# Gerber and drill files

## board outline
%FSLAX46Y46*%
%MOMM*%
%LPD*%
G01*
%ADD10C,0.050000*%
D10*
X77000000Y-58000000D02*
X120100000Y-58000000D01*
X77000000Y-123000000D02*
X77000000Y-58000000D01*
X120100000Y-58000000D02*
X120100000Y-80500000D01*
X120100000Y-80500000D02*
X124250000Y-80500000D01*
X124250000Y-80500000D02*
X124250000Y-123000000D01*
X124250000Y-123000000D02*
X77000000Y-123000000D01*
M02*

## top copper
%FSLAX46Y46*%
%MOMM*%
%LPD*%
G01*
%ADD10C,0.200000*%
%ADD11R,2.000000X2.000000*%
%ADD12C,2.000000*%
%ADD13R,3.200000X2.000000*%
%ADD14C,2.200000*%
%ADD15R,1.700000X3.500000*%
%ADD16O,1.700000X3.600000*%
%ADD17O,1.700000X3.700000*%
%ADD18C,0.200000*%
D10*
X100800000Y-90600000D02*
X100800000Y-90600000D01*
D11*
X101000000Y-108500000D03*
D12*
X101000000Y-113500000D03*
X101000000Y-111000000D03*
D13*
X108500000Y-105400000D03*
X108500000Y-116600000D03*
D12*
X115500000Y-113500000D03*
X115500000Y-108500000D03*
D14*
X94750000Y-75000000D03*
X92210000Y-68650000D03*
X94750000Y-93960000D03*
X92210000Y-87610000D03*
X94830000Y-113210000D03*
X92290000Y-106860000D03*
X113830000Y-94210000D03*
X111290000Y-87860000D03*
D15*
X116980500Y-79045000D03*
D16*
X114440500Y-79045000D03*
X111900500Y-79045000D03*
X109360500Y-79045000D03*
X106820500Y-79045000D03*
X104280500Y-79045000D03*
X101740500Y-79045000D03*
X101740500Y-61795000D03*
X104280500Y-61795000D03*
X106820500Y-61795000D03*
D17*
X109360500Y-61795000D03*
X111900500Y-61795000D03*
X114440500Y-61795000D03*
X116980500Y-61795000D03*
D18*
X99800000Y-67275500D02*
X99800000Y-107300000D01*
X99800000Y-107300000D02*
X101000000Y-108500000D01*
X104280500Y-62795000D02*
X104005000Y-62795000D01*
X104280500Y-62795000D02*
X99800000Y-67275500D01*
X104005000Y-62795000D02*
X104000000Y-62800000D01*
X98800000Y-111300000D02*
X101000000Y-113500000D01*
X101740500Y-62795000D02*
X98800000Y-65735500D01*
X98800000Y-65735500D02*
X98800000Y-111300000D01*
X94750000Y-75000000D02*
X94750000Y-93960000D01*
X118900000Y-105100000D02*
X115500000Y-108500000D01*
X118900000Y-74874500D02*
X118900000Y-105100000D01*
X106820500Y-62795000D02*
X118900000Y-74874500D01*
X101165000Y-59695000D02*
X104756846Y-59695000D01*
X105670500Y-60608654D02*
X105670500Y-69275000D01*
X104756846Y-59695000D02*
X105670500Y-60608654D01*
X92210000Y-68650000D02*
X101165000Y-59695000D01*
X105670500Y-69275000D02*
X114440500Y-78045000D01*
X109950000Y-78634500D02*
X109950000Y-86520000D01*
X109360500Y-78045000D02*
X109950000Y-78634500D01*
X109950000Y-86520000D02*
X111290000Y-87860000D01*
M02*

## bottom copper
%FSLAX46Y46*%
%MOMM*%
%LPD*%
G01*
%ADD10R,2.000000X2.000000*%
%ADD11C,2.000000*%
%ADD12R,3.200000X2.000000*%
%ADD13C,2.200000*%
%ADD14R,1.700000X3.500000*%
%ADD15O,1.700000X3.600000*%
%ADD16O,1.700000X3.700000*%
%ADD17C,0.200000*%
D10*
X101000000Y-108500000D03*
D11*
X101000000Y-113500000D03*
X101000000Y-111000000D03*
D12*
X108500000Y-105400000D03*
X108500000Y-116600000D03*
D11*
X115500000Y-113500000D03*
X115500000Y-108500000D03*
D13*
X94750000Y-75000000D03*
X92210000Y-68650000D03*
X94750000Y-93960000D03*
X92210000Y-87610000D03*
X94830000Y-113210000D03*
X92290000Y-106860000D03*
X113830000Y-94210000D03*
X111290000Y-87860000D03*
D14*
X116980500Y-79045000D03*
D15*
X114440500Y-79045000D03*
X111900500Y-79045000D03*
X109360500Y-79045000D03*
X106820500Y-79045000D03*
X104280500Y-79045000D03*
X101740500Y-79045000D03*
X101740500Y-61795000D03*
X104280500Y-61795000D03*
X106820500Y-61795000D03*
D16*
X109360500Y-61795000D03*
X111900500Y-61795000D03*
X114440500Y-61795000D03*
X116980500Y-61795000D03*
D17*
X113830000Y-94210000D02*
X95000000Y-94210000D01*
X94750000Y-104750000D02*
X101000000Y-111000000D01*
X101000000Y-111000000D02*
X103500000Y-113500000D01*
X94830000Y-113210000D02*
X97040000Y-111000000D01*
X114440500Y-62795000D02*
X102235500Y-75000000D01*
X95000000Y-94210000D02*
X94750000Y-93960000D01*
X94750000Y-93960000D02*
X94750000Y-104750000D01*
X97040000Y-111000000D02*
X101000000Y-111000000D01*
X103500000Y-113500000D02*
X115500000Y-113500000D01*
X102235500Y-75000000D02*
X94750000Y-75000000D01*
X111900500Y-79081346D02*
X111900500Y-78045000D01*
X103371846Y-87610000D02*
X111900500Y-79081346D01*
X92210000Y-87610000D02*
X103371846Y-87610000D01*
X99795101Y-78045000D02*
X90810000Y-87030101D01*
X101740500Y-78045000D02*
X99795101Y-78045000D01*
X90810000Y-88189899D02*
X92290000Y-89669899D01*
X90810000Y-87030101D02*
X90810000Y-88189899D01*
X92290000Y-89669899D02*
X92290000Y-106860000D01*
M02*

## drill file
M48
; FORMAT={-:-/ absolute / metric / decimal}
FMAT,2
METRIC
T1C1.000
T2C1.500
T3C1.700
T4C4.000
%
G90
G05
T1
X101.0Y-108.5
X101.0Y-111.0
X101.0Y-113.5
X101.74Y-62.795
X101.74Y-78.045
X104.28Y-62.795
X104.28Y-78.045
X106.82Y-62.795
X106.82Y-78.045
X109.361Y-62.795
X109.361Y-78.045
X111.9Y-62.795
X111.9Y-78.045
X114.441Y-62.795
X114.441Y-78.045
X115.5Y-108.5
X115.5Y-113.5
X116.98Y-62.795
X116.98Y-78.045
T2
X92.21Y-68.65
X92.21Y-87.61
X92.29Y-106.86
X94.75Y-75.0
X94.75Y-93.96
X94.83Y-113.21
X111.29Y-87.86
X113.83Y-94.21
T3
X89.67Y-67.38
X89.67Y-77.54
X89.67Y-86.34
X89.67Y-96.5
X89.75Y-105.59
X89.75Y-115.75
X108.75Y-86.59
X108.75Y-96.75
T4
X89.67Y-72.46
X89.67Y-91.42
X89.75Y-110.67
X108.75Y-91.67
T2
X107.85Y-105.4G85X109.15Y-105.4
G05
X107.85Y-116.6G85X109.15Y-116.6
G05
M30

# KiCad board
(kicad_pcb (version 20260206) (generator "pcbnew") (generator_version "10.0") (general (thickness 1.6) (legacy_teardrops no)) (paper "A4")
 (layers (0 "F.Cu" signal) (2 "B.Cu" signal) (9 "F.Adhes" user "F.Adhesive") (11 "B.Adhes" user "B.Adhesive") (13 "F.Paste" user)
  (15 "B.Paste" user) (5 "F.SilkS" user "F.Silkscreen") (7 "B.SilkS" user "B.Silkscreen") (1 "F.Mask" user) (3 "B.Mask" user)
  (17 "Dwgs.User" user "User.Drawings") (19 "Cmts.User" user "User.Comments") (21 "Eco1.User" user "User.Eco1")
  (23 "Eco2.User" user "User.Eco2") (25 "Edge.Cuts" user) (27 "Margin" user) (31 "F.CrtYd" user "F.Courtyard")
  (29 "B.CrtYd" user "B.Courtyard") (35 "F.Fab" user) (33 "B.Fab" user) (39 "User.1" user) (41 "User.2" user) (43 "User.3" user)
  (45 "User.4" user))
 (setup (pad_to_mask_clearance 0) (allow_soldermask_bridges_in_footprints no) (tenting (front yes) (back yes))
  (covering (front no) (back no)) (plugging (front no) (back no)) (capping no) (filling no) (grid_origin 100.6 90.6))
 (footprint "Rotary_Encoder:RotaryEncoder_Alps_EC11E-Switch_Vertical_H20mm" (layer "F.Cu") (at 101 108.5)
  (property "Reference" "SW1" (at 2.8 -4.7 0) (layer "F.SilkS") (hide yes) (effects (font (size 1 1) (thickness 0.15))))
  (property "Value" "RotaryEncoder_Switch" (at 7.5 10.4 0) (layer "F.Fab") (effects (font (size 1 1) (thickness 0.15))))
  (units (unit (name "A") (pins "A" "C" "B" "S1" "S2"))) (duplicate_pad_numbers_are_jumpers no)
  (pad "A" thru_hole rect (at 0 0) (size 2 2) (drill 1) (layers "*.Cu" "*.Mask") (remove_unused_layers no) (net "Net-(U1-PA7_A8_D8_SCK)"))
  (pad "B" thru_hole circle (at 0 5) (size 2 2) (drill 1) (layers "*.Cu" "*.Mask") (remove_unused_layers no) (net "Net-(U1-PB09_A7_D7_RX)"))
  (pad "C" thru_hole circle (at 0 2.5) (size 2 2) (drill 1) (layers "*.Cu" "*.Mask") (remove_unused_layers no) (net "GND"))
  (pad "MP" thru_hole rect (at 7.5 -3.1) (size 3.2 2) (drill oval 2.8 1.5) (layers "*.Cu" "*.Mask") (remove_unused_layers no))
  (pad "MP" thru_hole rect (at 7.5 8.1) (size 3.2 2) (drill oval 2.8 1.5) (layers "*.Cu" "*.Mask") (remove_unused_layers no))
  (pad "S1" thru_hole circle (at 14.5 5) (size 2 2) (drill 1) (layers "*.Cu" "*.Mask") (remove_unused_layers no) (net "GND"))
  (pad "S2" thru_hole circle (at 14.5 0) (size 2 2) (drill 1) (layers "*.Cu" "*.Mask") (remove_unused_layers no)
   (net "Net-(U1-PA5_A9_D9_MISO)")))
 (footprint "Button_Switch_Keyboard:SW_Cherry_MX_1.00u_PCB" (layer "F.Cu") (at 94.75 75 -90)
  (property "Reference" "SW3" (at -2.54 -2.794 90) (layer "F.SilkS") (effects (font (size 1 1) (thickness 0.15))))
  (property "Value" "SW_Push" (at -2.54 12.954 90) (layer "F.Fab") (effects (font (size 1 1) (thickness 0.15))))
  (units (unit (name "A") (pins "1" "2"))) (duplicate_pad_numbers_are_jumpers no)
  (pad "" np_thru_hole circle (at -7.62 5.08 270) (size 1.7 1.7) (drill 1.7) (layers "*.Cu" "*.Mask"))
  (pad "" np_thru_hole circle (at -2.54 5.08 270) (size 4 4) (drill 4) (layers "*.Cu" "*.Mask"))
  (pad "" np_thru_hole circle (at 2.54 5.08 270) (size 1.7 1.7) (drill 1.7) (layers "*.Cu" "*.Mask"))
  (pad "1" thru_hole circle (at 0 0 270) (size 2.2 2.2) (drill 1.5) (layers "*.Cu" "*.Mask") (remove_unused_layers no) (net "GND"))
  (pad "2" thru_hole circle (at -6.35 2.54 270) (size 2.2 2.2) (drill 1.5) (layers "*.Cu" "*.Mask") (remove_unused_layers no)
   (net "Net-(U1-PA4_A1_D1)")))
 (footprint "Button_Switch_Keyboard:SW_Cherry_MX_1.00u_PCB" (layer "F.Cu") (at 94.75 93.96 -90)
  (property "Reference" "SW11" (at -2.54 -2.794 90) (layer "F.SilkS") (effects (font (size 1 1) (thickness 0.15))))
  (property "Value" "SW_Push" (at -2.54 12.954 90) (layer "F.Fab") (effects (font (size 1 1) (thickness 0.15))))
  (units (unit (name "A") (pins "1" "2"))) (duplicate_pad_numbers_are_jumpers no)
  (pad "" np_thru_hole circle (at -7.62 5.08 270) (size 1.7 1.7) (drill 1.7) (layers "*.Cu" "*.Mask"))
  (pad "" np_thru_hole circle (at -2.54 5.08 270) (size 4 4) (drill 4) (layers "*.Cu" "*.Mask"))
  (pad "" np_thru_hole circle (at 2.54 5.08 270) (size 1.7 1.7) (drill 1.7) (layers "*.Cu" "*.Mask"))
  (pad "1" thru_hole circle (at 0 0 270) (size 2.2 2.2) (drill 1.5) (layers "*.Cu" "*.Mask") (remove_unused_layers no) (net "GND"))
  (pad "2" thru_hole circle (at -6.35 2.54 270) (size 2.2 2.2) (drill 1.5) (layers "*.Cu" "*.Mask") (remove_unused_layers no)
   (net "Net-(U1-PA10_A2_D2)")))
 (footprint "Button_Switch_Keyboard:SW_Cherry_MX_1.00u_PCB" (layer "F.Cu") (at 94.83 113.21 -90)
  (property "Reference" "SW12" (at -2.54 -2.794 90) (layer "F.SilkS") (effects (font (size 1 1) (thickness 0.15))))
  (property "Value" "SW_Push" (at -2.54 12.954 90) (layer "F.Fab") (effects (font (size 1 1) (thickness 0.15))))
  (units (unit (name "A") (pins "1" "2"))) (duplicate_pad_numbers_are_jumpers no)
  (pad "" np_thru_hole circle (at -7.62 5.08 270) (size 1.7 1.7) (drill 1.7) (layers "*.Cu" "*.Mask"))
  (pad "" np_thru_hole circle (at -2.54 5.08 270) (size 4 4) (drill 4) (layers "*.Cu" "*.Mask"))
  (pad "" np_thru_hole circle (at 2.54 5.08 270) (size 1.7 1.7) (drill 1.7) (layers "*.Cu" "*.Mask"))
  (pad "1" thru_hole circle (at 0 0 270) (size 2.2 2.2) (drill 1.5) (layers "*.Cu" "*.Mask") (remove_unused_layers no) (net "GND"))
  (pad "2" thru_hole circle (at -6.35 2.54 270) (size 2.2 2.2) (drill 1.5) (layers "*.Cu" "*.Mask") (remove_unused_layers no)
   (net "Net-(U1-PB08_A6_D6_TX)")))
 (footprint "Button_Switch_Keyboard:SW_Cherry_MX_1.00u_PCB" (layer "F.Cu") (at 113.83 94.21 -90)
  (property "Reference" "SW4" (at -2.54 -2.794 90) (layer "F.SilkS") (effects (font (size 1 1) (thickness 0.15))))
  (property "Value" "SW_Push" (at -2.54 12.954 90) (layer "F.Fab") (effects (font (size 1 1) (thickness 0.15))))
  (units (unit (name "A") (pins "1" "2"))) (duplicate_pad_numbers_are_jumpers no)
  (pad "" np_thru_hole circle (at -7.62 5.08 270) (size 1.7 1.7) (drill 1.7) (layers "*.Cu" "*.Mask"))
  (pad "" np_thru_hole circle (at -2.54 5.08 270) (size 4 4) (drill 4) (layers "*.Cu" "*.Mask"))
  (pad "" np_thru_hole circle (at 2.54 5.08 270) (size 1.7 1.7) (drill 1.7) (layers "*.Cu" "*.Mask"))
  (pad "1" thru_hole circle (at 0 0 270) (size 2.2 2.2) (drill 1.5) (layers "*.Cu" "*.Mask") (remove_unused_layers no) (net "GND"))
  (pad "2" thru_hole circle (at -6.35 2.54 270) (size 2.2 2.2) (drill 1.5) (layers "*.Cu" "*.Mask") (remove_unused_layers no)
   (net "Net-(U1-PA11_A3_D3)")))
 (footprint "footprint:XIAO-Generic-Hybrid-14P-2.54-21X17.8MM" (layer "B.Cu") (at 109.3605 70.42 90)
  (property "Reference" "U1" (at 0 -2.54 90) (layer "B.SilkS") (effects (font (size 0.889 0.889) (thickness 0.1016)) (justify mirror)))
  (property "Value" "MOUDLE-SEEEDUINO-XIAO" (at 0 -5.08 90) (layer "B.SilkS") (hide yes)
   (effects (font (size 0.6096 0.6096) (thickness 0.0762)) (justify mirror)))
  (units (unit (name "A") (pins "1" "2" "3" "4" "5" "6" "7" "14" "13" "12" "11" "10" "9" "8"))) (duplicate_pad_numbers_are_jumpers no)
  (pad "1" thru_hole rect (at -7.625 7.62 90) (size 3.5 1.7) (drill 1 (offset -1 0)) (layers "*.Cu" "*.Mask") (remove_unused_layers no)
   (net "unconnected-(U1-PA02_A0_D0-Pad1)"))
  (pad "2" thru_hole oval (at -7.625 5.08 90) (size 3.6 1.7) (drill 1 (offset -1 0)) (layers "*.Cu" "*.Mask") (remove_unused_layers no)
   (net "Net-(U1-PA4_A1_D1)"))
  (pad "3" thru_hole oval (at -7.625 2.54 90) (size 3.6 1.7) (drill 1 (offset -1 0)) (layers "*.Cu" "*.Mask") (remove_unused_layers no)
   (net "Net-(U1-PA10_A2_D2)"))
  (pad "4" thru_hole oval (at -7.625 0 90) (size 3.6 1.7) (drill 1 (offset -1 0)) (layers "*.Cu" "*.Mask") (remove_unused_layers no)
   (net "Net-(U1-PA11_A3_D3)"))
  (pad "5" thru_hole oval (at -7.625 -2.54 90) (size 3.6 1.7) (drill 1 (offset -1 0)) (layers "*.Cu" "*.Mask") (remove_unused_layers no)
   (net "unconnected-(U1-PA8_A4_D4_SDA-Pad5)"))
  (pad "6" thru_hole oval (at -7.625 -5.08 270) (size 3.6 1.7) (drill 1 (offset 1 0)) (layers "*.Cu" "*.Mask") (remove_unused_layers no)
   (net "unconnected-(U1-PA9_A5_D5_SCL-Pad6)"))
  (pad "7" thru_hole oval (at -7.625 -7.62 90) (size 3.6 1.7) (drill 1 (offset -1 0)) (layers "*.Cu" "*.Mask") (remove_unused_layers no)
   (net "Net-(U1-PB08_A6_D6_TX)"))
  (pad "8" thru_hole oval (at 7.625 -7.62 90) (size 3.6 1.7) (drill 1 (offset 1 0)) (layers "*.Cu" "*.Mask") (remove_unused_layers no)
   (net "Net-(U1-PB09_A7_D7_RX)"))
  (pad "9" thru_hole oval (at 7.625 -5.08 90) (size 3.6 1.7) (drill 1 (offset 1 0)) (layers "*.Cu" "*.Mask") (remove_unused_layers no)
   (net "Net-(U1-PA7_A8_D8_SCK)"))
  (pad "10" thru_hole oval (at 7.625 -2.54 90) (size 3.6 1.7) (drill 1 (offset 1 0)) (layers "*.Cu" "*.Mask") (remove_unused_layers no)
   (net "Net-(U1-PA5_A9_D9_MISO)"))
  (pad "11" thru_hole oval (at 7.625 0 90) (size 3.7 1.7) (drill 1 (offset 1 0)) (layers "*.Cu" "*.Mask") (remove_unused_layers no)
   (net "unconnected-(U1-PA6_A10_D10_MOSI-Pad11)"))
  (pad "12" thru_hole oval (at 7.625 2.54 90) (size 3.7 1.7) (drill 1 (offset 1 0)) (layers "*.Cu" "*.Mask") (remove_unused_layers no)
   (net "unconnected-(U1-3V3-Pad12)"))
  (pad "13" thru_hole oval (at 7.625 5.08 90) (size 3.7 1.7) (drill 1 (offset 1 0)) (layers "*.Cu" "*.Mask") (remove_unused_layers no)
   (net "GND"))
  (pad "14" thru_hole oval (at 7.625 7.62 90) (size 3.7 1.7) (drill 1 (offset 1 0)) (layers "*.Cu" "*.Mask") (remove_unused_layers no)
   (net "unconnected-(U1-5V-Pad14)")))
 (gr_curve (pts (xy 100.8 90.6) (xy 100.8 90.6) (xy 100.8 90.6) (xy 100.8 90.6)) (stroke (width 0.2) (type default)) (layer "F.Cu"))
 (gr_line (start 77 58) (end 120.1 58) (stroke (width 0.05) (type default)) (layer "Edge.Cuts"))
 (gr_line (start 77 123) (end 77 58) (stroke (width 0.05) (type default)) (layer "Edge.Cuts"))
 (gr_line (start 120.1 58) (end 120.1 80.5) (stroke (width 0.05) (type default)) (layer "Edge.Cuts"))
 (gr_line (start 120.1 80.5) (end 124.25 80.5) (stroke (width 0.05) (type default)) (layer "Edge.Cuts"))
 (gr_line (start 124.25 80.5) (end 124.25 123) (stroke (width 0.05) (type default)) (layer "Edge.Cuts"))
 (gr_line (start 124.25 123) (end 77 123) (stroke (width 0.05) (type default)) (layer "Edge.Cuts"))
 (segment (start 99.8 67.2755) (end 99.8 107.3) (width 0.2) (layer "F.Cu") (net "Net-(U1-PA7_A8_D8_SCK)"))
 (segment (start 99.8 107.3) (end 101 108.5) (width 0.2) (layer "F.Cu") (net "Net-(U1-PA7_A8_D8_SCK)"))
 (segment (start 104.2805 62.795) (end 104.005 62.795) (width 0.2) (layer "F.Cu") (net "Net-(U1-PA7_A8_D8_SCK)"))
 (segment (start 104.2805 62.795) (end 99.8 67.2755) (width 0.2) (layer "F.Cu") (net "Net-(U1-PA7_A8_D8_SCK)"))
 (segment (start 104.005 62.795) (end 104 62.8) (width 0.2) (layer "F.Cu") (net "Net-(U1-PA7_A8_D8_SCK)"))
 (segment (start 98.8 111.3) (end 101 113.5) (width 0.2) (layer "F.Cu") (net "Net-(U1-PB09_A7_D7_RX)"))
 (segment (start 101.7405 62.795) (end 98.8 65.7355) (width 0.2) (layer "F.Cu") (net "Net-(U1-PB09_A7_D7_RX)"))
 (segment (start 98.8 65.7355) (end 98.8 111.3) (width 0.2) (layer "F.Cu") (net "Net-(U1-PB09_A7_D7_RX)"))
 (segment (start 94.75 75) (end 94.75 93.96) (width 0.2) (layer "F.Cu") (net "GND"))
 (segment (start 113.83 94.21) (end 95 94.21) (width 0.2) (layer "B.Cu") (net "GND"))
 (segment (start 94.75 104.75) (end 101 111) (width 0.2) (layer "B.Cu") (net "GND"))
 (segment (start 101 111) (end 103.5 113.5) (width 0.2) (layer "B.Cu") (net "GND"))
 (segment (start 94.83 113.21) (end 97.04 111) (width 0.2) (layer "B.Cu") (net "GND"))
 (segment (start 114.4405 62.795) (end 102.2355 75) (width 0.2) (layer "B.Cu") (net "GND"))
 (segment (start 95 94.21) (end 94.75 93.96) (width 0.2) (layer "B.Cu") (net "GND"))
 (segment (start 94.75 93.96) (end 94.75 104.75) (width 0.2) (layer "B.Cu") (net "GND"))
 (segment (start 97.04 111) (end 101 111) (width 0.2) (layer "B.Cu") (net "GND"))
 (segment (start 103.5 113.5) (end 115.5 113.5) (width 0.2) (layer "B.Cu") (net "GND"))
 (segment (start 102.2355 75) (end 94.75 75) (width 0.2) (layer "B.Cu") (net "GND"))
 (segment (start 118.9 105.1) (end 115.5 108.5) (width 0.2) (layer "F.Cu") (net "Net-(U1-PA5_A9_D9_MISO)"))
 (segment (start 118.9 74.8745) (end 118.9 105.1) (width 0.2) (layer "F.Cu") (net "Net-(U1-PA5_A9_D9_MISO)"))
 (segment (start 106.8205 62.795) (end 118.9 74.8745) (width 0.2) (layer "F.Cu") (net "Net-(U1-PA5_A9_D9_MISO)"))
 (segment (start 101.165 59.695) (end 104.756846 59.695) (width 0.2) (layer "F.Cu") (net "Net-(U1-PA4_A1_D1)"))
 (segment (start 105.6705 60.608654) (end 105.6705 69.275) (width 0.2) (layer "F.Cu") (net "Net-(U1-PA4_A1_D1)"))
 (segment (start 104.756846 59.695) (end 105.6705 60.608654) (width 0.2) (layer "F.Cu") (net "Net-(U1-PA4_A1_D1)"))
 (segment (start 92.21 68.65) (end 101.165 59.695) (width 0.2) (layer "F.Cu") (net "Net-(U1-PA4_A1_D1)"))
 (segment (start 105.6705 69.275) (end 114.4405 78.045) (width 0.2) (layer "F.Cu") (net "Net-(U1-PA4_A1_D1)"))
 (segment (start 111.9005 79.081346) (end 111.9005 78.045) (width 0.2) (layer "B.Cu") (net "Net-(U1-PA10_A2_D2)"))
 (segment (start 103.371846 87.61) (end 111.9005 79.081346) (width 0.2) (layer "B.Cu") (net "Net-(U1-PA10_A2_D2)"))
 (segment (start 92.21 87.61) (end 103.371846 87.61) (width 0.2) (layer "B.Cu") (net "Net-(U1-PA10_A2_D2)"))
 (segment (start 99.795101 78.045) (end 90.81 87.030101) (width 0.2) (layer "B.Cu") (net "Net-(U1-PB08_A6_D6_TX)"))
 (segment (start 101.7405 78.045) (end 99.795101 78.045) (width 0.2) (layer "B.Cu") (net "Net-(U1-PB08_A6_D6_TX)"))
 (segment (start 90.81 88.189899) (end 92.29 89.669899) (width 0.2) (layer "B.Cu") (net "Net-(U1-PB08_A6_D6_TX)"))
 (segment (start 90.81 87.030101) (end 90.81 88.189899) (width 0.2) (layer "B.Cu") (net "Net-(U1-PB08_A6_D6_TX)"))
 (segment (start 92.29 89.669899) (end 92.29 106.86) (width 0.2) (layer "B.Cu") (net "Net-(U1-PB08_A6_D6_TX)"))
 (segment (start 109.95 78.6345) (end 109.95 86.52) (width 0.2) (layer "F.Cu") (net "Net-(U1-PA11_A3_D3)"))
 (segment (start 109.3605 78.045) (end 109.95 78.6345) (width 0.2) (layer "F.Cu") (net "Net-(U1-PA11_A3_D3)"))
 (segment (start 109.95 86.52) (end 111.29 87.86) (width 0.2) (layer "F.Cu") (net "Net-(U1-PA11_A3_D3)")))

